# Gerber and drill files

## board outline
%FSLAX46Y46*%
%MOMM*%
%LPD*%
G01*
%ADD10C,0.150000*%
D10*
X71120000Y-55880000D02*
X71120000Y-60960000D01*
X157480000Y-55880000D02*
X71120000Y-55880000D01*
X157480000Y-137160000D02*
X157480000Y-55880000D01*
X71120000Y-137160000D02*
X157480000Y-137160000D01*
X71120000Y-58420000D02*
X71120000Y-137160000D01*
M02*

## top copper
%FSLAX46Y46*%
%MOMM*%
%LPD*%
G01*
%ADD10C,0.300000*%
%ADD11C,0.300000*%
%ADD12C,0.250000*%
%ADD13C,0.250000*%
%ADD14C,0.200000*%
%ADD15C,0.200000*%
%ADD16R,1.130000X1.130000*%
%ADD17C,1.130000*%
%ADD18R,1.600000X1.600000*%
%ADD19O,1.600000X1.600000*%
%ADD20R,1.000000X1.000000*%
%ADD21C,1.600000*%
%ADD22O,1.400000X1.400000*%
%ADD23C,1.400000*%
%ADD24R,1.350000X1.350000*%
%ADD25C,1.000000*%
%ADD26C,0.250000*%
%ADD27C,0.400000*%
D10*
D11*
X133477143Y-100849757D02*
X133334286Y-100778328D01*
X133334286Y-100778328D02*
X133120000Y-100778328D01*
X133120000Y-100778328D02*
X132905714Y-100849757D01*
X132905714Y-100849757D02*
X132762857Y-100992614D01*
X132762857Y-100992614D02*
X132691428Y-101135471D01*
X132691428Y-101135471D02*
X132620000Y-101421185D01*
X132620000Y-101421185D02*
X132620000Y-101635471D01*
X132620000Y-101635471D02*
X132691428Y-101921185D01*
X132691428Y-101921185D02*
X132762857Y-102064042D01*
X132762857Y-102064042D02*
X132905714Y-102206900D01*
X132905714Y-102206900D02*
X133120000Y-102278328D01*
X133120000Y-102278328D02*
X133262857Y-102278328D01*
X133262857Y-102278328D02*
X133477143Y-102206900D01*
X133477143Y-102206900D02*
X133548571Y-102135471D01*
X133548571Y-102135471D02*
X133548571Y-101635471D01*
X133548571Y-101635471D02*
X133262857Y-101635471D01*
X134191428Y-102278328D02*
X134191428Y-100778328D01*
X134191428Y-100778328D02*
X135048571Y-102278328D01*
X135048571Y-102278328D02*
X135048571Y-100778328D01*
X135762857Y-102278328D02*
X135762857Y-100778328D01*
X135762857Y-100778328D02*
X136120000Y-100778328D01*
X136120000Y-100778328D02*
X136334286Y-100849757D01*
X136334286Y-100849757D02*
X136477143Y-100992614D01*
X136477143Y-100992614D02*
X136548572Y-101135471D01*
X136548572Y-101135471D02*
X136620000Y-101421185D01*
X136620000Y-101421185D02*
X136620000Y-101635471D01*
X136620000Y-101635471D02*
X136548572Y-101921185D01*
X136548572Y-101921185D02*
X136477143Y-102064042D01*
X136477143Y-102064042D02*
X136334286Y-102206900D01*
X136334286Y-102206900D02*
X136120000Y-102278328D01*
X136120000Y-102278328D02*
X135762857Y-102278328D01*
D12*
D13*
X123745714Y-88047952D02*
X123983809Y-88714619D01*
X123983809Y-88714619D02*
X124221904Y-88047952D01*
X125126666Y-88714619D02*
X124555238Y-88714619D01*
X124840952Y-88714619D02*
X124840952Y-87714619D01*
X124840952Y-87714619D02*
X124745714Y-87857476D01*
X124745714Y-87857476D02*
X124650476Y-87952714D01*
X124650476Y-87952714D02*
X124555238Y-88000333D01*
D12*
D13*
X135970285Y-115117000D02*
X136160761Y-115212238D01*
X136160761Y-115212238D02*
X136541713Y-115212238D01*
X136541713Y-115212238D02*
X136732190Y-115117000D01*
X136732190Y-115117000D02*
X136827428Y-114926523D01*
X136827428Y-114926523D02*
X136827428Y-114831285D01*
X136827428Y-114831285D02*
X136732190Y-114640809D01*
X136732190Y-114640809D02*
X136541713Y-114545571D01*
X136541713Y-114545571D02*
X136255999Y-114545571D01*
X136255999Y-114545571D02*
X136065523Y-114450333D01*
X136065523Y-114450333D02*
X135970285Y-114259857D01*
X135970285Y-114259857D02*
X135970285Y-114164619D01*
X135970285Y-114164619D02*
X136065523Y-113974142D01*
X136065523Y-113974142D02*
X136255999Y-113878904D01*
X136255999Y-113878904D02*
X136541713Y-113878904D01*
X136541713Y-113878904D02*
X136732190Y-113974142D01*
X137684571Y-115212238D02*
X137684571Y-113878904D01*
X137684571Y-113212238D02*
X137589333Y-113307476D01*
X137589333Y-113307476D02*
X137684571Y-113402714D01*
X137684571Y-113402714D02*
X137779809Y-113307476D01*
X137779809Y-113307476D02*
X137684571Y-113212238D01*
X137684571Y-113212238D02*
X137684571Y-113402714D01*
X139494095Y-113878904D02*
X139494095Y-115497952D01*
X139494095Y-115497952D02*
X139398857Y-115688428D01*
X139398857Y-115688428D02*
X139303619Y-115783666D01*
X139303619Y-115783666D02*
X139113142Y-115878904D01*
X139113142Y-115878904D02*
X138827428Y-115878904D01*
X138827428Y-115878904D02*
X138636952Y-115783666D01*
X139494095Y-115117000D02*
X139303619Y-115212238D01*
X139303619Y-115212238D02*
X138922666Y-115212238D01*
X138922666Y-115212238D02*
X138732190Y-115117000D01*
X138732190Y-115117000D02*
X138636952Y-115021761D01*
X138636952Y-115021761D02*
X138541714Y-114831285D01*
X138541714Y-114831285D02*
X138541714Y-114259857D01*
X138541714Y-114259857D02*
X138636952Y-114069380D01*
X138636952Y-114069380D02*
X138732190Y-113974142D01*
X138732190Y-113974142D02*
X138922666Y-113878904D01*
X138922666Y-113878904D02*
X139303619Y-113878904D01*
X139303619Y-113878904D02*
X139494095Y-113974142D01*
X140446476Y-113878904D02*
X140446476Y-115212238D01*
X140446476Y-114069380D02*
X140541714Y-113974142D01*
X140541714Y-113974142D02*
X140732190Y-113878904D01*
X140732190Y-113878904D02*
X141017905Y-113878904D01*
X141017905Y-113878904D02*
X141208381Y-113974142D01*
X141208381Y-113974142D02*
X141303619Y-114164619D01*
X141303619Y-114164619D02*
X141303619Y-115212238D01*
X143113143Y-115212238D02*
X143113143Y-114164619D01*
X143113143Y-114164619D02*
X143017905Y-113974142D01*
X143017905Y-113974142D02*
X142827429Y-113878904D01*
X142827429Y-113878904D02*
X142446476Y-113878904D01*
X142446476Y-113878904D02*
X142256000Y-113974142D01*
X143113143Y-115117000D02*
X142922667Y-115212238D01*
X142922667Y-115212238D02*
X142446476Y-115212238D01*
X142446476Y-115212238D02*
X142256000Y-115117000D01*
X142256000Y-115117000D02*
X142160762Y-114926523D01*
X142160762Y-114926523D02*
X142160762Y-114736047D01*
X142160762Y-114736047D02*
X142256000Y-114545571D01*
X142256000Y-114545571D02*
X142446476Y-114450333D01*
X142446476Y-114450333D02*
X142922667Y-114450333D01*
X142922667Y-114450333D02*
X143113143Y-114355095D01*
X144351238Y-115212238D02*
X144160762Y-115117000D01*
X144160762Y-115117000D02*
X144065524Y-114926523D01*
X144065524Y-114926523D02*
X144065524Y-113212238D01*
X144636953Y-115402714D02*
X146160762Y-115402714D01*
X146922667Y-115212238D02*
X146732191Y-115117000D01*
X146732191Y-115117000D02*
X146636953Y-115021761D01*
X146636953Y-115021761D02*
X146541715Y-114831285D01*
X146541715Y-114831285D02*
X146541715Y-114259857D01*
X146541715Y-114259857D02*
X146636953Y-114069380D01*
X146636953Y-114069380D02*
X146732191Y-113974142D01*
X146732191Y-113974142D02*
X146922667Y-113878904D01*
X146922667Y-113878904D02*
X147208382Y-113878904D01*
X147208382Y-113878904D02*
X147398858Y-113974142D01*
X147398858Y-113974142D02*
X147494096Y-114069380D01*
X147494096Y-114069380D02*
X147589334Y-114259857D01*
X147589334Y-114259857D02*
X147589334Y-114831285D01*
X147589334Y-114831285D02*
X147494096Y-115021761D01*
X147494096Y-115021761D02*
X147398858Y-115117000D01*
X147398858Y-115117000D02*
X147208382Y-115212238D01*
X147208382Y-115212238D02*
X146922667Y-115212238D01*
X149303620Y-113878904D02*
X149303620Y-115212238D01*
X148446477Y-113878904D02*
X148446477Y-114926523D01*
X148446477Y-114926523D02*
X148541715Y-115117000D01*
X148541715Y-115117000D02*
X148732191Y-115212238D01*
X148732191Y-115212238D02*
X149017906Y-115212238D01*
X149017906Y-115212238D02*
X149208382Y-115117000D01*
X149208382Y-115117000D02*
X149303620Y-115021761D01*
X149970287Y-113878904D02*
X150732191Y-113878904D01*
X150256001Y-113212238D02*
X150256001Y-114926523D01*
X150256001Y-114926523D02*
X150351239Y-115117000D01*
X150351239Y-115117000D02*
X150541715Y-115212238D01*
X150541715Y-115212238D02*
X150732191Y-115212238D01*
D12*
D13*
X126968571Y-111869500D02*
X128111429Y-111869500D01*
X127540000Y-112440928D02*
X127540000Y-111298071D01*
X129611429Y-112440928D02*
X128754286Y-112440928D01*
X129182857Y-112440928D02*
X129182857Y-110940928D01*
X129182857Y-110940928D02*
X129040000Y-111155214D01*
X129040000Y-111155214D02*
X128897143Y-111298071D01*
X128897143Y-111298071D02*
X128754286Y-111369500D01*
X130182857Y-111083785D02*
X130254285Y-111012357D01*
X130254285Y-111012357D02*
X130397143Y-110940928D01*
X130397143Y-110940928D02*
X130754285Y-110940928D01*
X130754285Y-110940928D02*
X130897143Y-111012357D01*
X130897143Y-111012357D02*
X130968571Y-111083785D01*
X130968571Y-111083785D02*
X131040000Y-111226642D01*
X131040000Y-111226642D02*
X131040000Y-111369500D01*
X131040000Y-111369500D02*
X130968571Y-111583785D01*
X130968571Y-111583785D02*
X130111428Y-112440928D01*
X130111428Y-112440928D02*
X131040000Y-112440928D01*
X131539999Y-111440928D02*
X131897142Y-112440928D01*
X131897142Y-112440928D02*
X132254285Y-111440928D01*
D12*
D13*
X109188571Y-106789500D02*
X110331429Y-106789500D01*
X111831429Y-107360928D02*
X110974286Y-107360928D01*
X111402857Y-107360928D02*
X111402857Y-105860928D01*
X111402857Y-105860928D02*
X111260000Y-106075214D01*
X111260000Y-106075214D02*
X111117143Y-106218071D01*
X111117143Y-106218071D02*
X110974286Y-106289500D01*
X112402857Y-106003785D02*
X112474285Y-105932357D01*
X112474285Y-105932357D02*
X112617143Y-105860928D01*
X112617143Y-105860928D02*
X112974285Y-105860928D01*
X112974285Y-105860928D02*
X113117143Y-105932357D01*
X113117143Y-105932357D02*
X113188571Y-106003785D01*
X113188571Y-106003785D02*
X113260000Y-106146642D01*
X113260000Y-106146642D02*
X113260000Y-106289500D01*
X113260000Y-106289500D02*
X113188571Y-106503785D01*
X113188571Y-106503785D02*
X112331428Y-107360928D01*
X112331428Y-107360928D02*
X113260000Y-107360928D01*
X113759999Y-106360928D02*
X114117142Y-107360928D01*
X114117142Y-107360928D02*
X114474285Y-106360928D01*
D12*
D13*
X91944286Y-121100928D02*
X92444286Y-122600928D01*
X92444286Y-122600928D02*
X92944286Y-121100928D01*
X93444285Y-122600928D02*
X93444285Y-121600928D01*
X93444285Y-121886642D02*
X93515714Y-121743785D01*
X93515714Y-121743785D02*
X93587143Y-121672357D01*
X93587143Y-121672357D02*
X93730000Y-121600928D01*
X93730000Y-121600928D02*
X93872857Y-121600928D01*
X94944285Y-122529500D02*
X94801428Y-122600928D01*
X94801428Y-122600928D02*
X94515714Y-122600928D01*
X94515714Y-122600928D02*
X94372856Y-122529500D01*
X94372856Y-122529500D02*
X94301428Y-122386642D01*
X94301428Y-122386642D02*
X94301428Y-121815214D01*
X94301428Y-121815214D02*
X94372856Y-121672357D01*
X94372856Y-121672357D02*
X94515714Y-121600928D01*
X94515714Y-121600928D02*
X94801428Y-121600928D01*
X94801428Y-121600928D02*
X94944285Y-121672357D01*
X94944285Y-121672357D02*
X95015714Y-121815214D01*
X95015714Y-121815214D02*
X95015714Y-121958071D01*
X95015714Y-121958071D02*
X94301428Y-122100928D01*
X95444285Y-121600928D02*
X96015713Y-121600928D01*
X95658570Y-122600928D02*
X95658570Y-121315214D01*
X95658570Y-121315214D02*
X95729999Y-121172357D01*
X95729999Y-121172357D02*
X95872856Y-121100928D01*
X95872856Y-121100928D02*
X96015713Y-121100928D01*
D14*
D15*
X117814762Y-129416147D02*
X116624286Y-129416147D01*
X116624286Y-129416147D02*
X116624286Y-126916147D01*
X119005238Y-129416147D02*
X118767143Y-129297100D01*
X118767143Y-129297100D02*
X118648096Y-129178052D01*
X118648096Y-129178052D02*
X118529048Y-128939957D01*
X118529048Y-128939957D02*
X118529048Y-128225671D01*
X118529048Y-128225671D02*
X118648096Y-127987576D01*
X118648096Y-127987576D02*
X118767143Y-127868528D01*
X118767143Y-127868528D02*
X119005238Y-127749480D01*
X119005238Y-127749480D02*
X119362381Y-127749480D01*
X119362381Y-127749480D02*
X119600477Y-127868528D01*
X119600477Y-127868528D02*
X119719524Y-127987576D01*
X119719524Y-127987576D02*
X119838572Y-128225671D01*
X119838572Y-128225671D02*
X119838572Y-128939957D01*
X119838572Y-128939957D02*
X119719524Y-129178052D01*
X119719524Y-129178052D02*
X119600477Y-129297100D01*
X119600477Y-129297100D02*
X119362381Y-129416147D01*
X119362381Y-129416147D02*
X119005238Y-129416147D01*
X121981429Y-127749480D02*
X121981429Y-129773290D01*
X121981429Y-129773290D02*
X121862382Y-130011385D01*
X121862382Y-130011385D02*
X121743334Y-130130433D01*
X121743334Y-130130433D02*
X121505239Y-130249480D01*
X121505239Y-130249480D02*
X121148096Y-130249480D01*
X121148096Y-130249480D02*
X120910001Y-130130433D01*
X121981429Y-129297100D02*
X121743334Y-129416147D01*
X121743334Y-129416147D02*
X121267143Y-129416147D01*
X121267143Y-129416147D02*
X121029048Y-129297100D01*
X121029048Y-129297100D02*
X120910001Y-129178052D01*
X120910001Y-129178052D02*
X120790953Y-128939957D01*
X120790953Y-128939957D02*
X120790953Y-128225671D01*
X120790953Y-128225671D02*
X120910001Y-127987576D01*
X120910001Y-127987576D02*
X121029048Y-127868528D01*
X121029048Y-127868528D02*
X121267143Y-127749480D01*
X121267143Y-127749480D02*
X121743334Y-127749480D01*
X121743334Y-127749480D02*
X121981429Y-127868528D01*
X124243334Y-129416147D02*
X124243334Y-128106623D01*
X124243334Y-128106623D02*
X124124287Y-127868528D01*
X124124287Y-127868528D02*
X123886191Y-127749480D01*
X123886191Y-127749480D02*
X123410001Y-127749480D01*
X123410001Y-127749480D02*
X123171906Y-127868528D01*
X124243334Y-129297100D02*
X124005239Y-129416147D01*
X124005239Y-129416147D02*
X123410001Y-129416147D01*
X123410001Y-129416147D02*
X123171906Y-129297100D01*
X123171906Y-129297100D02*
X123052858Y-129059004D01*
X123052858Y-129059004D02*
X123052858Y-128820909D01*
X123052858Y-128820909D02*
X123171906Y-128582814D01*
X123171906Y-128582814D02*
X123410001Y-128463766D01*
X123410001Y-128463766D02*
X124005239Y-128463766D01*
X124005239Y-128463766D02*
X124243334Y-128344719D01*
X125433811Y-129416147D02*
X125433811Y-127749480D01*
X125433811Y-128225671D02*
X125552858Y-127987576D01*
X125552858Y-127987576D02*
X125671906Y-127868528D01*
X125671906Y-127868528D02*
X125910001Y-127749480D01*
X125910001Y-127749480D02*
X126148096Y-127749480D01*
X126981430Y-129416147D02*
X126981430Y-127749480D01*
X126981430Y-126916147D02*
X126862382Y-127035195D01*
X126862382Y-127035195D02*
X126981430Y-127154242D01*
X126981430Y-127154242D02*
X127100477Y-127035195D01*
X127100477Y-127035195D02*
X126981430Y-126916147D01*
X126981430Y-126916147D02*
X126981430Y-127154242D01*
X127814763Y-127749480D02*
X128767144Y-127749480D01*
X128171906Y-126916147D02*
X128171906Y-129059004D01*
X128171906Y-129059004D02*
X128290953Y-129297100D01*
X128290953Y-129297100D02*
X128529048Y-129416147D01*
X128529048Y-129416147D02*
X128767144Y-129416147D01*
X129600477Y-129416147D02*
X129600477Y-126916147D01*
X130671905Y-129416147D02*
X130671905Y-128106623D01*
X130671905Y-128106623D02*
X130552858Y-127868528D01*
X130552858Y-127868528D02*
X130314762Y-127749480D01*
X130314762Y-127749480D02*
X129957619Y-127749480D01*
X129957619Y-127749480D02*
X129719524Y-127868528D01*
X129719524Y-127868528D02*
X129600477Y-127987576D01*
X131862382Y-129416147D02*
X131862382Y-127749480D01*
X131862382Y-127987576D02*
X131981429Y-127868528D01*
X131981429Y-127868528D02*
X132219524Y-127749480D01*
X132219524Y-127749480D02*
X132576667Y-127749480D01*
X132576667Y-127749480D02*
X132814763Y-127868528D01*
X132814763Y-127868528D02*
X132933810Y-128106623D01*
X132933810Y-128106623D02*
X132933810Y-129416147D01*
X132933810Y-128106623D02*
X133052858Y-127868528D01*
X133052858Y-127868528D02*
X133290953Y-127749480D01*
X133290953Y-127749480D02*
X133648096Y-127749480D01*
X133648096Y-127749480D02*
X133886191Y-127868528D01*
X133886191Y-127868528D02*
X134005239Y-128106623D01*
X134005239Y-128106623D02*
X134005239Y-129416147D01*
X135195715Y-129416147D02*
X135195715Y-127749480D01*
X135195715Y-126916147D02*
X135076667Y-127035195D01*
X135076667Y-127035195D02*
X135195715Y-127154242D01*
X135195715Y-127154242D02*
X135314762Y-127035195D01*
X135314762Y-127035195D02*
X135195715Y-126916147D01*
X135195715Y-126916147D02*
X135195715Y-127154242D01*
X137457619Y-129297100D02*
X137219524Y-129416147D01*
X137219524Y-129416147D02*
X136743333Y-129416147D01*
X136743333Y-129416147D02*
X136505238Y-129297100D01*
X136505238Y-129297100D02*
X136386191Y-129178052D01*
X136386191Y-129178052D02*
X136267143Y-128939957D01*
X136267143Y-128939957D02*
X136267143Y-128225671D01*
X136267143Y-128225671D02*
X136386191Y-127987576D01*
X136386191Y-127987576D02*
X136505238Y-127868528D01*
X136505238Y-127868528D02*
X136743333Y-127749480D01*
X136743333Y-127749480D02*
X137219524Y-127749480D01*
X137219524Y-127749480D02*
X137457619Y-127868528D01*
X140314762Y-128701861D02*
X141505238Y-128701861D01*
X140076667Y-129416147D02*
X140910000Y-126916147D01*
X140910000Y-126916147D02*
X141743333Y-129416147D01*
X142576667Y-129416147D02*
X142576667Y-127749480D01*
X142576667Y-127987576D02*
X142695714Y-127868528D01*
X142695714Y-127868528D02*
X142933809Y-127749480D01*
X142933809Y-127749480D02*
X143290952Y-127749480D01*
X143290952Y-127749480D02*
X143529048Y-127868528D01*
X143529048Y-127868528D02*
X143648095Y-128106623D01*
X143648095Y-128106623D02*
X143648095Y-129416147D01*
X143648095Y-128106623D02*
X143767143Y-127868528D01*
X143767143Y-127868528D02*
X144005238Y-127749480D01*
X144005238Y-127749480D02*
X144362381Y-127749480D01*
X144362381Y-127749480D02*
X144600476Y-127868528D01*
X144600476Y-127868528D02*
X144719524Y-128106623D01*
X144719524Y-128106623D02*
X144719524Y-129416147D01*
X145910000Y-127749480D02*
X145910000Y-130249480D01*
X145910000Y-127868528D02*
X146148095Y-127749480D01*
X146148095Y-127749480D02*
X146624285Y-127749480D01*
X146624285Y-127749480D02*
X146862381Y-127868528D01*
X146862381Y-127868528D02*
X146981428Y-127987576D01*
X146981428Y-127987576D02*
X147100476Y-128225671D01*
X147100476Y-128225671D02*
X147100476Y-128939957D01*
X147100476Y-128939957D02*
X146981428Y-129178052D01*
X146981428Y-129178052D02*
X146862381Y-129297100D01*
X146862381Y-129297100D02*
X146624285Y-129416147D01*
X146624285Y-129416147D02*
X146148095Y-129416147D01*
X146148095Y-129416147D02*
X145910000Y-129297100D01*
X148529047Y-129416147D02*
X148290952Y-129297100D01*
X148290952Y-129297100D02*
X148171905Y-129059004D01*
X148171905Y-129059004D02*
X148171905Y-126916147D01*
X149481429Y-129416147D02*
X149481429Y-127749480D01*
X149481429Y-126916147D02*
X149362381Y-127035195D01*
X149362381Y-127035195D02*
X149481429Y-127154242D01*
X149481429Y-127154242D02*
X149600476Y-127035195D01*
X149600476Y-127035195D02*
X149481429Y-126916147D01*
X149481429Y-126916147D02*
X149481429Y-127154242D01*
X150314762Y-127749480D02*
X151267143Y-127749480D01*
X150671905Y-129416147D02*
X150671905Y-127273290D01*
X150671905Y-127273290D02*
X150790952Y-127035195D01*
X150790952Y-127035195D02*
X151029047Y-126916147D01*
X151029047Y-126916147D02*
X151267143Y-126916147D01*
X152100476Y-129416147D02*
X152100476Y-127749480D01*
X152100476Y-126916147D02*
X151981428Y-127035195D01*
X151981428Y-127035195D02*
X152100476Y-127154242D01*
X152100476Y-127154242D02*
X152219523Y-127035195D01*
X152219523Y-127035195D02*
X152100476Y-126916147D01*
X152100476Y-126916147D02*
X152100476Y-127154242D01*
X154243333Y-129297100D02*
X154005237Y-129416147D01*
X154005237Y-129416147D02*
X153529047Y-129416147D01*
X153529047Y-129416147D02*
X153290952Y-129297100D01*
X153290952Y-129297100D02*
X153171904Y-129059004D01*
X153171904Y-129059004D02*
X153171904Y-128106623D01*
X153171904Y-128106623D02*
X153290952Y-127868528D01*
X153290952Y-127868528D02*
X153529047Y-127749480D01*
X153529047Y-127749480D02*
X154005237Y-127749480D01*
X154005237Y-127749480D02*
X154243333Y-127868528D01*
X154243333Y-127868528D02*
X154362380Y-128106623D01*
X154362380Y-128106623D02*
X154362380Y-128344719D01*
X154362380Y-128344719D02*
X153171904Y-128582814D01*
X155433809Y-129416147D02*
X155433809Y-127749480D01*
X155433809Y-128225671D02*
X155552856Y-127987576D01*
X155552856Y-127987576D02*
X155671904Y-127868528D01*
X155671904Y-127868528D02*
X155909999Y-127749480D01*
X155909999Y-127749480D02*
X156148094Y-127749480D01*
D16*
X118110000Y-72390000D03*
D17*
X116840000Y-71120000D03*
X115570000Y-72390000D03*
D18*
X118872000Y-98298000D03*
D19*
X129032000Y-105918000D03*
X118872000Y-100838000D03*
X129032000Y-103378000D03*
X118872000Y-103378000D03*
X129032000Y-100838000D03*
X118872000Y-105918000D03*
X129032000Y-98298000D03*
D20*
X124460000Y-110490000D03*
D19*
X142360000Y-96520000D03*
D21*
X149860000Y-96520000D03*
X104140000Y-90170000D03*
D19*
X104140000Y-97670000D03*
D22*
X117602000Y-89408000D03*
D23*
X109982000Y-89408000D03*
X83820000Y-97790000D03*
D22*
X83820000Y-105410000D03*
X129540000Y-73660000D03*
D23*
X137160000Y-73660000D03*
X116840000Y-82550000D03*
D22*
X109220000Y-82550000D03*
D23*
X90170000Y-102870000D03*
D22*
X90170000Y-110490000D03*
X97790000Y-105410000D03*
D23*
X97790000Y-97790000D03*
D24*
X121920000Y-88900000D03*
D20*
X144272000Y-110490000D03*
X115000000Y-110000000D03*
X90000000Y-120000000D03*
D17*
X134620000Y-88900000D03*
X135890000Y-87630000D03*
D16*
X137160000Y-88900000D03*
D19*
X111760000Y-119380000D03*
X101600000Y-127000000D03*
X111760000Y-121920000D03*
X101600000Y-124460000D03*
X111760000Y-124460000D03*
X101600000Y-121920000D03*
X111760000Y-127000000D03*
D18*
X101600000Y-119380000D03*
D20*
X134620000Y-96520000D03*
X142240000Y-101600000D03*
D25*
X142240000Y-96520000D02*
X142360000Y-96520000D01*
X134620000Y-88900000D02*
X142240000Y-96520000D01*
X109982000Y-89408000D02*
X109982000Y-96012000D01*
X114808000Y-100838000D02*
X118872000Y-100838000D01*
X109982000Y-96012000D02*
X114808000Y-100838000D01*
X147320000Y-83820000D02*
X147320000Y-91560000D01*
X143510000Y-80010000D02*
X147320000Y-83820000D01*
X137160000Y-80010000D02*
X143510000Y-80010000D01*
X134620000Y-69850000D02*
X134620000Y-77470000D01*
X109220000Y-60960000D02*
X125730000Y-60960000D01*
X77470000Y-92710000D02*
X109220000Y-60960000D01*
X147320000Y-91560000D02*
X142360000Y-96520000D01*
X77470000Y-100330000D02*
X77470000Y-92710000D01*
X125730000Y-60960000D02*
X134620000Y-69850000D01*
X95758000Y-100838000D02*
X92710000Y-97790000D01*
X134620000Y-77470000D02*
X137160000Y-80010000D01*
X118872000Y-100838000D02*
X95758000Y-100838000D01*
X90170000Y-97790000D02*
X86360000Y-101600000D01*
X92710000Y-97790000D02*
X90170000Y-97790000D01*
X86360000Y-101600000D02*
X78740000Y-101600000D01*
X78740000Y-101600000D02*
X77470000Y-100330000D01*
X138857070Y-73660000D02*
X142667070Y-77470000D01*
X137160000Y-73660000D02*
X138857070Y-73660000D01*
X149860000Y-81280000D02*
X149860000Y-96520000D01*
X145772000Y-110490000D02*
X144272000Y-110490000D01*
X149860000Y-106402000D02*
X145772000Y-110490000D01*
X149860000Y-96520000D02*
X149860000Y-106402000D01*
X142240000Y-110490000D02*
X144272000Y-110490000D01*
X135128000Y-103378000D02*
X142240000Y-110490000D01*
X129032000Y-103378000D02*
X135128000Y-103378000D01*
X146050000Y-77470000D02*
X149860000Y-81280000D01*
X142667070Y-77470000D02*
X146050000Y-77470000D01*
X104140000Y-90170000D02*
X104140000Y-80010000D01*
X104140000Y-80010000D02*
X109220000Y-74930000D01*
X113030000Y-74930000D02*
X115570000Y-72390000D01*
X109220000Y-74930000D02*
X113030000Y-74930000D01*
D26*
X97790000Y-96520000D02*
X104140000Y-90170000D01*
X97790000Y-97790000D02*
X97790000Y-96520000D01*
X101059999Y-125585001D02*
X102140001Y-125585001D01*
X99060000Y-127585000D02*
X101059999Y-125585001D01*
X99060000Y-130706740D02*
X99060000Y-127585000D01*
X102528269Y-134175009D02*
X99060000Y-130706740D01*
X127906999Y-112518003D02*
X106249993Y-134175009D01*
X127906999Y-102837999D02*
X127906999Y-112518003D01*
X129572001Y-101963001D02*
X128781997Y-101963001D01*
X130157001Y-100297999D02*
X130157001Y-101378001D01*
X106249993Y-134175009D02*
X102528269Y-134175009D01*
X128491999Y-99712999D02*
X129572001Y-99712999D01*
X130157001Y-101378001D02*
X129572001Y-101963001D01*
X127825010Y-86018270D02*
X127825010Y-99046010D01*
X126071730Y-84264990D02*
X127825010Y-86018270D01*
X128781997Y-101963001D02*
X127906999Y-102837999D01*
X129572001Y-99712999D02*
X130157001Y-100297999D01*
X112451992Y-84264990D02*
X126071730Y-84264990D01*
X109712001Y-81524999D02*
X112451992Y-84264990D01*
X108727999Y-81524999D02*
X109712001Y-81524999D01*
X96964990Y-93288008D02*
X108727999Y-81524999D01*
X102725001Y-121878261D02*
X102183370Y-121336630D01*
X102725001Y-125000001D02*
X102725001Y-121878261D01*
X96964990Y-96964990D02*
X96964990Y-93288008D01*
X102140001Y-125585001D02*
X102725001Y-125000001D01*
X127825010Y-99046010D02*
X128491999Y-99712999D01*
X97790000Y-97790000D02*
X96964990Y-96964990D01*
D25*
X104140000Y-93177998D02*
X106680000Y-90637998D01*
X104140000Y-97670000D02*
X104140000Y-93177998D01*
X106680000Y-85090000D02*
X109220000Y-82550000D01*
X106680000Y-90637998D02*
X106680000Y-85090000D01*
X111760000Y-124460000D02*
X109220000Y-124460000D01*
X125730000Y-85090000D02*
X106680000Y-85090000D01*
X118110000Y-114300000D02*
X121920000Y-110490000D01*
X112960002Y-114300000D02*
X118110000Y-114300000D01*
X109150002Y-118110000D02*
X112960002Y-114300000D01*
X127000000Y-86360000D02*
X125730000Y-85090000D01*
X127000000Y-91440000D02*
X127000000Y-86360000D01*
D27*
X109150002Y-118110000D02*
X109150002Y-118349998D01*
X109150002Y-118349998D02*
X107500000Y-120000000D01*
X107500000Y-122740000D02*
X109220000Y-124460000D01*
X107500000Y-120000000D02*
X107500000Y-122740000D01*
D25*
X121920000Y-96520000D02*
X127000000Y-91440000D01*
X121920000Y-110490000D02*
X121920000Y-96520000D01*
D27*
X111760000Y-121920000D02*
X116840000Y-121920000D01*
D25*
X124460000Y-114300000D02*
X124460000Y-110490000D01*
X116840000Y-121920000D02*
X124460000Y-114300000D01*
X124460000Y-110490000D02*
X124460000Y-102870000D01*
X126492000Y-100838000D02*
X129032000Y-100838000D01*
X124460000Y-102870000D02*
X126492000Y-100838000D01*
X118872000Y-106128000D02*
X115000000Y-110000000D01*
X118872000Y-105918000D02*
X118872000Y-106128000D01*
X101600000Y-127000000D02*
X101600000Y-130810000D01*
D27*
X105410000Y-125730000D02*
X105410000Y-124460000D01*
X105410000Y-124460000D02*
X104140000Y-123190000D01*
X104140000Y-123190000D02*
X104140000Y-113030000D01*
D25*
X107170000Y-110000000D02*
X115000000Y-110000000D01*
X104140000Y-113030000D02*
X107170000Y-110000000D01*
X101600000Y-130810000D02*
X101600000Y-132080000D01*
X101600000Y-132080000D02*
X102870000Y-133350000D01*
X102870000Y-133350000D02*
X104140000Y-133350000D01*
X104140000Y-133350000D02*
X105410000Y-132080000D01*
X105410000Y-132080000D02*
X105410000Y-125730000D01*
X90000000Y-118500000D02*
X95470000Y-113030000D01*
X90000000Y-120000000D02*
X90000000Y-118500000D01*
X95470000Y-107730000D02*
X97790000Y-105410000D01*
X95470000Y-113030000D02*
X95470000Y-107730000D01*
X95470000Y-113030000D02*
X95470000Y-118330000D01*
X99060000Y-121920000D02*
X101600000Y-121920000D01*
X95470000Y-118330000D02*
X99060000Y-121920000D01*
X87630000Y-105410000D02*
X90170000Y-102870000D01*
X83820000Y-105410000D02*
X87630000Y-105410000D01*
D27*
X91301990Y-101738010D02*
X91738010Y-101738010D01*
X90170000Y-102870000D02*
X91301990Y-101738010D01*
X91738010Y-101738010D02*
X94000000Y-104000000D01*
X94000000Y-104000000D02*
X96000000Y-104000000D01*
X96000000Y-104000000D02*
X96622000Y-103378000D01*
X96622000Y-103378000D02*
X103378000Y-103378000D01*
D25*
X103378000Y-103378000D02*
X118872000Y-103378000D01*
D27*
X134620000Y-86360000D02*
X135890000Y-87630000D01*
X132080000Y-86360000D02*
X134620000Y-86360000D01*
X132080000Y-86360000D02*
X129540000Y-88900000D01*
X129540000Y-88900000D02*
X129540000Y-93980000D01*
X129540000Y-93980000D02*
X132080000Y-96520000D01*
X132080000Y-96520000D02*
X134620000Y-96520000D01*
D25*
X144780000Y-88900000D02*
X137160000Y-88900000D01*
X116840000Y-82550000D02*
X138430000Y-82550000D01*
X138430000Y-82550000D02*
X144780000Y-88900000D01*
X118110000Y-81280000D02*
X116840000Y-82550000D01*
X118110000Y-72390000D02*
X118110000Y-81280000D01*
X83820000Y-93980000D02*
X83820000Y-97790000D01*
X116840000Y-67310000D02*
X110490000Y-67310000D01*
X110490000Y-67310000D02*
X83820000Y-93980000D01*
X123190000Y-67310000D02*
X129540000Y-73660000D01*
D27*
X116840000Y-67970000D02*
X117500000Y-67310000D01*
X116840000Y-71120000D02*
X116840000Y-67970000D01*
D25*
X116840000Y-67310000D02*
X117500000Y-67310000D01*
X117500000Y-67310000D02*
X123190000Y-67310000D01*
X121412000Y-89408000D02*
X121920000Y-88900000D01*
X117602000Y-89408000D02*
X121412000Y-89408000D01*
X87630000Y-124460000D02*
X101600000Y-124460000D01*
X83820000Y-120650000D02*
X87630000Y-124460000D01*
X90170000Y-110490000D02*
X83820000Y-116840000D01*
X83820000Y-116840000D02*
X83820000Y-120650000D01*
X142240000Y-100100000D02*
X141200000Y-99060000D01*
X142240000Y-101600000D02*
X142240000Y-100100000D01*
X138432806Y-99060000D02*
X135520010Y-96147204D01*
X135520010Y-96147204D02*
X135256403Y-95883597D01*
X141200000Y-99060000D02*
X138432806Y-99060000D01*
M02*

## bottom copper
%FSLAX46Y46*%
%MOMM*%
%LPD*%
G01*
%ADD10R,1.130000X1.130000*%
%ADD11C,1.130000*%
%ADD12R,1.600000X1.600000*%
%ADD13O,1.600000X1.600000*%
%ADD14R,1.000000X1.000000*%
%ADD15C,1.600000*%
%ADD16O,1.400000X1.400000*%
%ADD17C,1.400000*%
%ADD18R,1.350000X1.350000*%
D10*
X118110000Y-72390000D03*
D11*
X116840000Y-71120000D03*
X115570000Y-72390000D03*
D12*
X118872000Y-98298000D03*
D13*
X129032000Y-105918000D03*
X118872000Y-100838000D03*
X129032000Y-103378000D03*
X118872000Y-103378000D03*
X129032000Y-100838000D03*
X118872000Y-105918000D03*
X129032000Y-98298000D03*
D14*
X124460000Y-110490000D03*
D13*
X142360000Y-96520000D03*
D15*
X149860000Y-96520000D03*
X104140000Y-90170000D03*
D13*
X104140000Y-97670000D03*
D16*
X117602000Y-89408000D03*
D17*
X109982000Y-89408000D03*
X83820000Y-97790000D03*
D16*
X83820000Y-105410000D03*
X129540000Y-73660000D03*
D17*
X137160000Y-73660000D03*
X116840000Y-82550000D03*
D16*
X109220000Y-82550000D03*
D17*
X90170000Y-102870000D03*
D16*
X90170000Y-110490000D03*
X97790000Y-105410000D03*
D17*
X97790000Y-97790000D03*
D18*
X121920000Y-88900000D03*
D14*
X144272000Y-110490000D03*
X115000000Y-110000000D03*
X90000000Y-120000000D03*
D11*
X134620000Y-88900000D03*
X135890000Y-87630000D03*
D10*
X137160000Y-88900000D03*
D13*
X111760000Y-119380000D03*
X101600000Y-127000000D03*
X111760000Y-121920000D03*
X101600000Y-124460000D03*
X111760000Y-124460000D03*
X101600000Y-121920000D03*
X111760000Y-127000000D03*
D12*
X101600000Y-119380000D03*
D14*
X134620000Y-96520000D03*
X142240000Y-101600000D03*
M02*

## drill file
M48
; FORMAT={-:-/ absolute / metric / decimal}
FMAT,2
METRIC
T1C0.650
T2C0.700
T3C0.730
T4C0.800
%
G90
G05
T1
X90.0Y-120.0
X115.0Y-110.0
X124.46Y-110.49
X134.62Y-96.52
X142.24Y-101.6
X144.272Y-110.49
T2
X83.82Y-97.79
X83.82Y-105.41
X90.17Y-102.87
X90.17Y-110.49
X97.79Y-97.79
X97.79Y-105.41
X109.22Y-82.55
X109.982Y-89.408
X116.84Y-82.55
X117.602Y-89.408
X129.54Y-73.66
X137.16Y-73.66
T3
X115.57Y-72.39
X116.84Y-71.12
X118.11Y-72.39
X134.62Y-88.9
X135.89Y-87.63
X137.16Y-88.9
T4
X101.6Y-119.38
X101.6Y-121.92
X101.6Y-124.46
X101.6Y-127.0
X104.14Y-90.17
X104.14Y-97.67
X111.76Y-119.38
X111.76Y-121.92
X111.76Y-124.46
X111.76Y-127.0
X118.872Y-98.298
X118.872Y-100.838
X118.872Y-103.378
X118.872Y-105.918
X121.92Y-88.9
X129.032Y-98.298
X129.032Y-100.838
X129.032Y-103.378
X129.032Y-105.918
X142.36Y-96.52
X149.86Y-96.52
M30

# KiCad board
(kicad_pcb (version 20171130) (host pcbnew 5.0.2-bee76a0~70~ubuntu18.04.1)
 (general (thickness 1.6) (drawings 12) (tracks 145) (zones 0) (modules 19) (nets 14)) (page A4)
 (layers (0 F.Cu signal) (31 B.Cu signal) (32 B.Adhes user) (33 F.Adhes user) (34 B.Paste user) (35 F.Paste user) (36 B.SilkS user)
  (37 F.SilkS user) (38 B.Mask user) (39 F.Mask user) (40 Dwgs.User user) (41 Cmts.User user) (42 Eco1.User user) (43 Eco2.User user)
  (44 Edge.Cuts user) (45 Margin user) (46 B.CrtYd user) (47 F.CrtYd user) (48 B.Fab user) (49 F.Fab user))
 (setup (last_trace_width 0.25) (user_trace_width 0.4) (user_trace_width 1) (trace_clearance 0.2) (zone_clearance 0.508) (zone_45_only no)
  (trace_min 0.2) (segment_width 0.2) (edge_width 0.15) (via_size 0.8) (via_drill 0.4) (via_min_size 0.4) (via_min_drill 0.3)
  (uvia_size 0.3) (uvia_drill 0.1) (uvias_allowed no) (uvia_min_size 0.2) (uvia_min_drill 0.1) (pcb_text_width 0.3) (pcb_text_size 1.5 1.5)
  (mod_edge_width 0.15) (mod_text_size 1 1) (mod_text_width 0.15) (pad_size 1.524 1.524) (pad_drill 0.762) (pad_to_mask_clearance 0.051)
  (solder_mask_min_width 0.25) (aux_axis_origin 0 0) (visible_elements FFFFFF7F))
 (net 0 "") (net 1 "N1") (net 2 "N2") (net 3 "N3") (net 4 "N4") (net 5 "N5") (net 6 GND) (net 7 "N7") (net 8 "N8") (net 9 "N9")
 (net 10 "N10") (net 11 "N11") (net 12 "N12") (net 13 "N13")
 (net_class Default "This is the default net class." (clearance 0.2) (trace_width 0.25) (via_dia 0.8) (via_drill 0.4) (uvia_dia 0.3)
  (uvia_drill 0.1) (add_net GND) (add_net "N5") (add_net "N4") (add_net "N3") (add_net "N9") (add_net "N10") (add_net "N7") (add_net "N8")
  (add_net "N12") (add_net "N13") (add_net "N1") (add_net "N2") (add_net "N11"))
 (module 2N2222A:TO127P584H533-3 (layer F.Cu) (at 116.84 72.39 180)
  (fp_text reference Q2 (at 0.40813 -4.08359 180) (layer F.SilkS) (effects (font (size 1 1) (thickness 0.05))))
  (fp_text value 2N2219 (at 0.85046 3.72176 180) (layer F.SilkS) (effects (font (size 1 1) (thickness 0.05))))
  (pad 1 thru_hole rect (at -1.27 0 180) (size 1.13 1.13) (drill 0.73) (layers *.Cu *.Mask) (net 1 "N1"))
  (pad 2 thru_hole circle (at 0 1.27 180) (size 1.13 1.13) (drill 0.73) (layers *.Cu *.Mask) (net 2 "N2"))
  (pad 3 thru_hole circle (at 1.27 0 180) (size 1.13 1.13) (drill 0.73) (layers *.Cu *.Mask) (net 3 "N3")))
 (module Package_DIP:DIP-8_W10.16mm (layer F.Cu) (at 118.872 98.298)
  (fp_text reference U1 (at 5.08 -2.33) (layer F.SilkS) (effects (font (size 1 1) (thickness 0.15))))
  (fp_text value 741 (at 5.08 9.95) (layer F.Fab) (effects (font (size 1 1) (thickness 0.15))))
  (pad 1 thru_hole rect (at 0 0) (size 1.6 1.6) (drill 0.8) (layers *.Cu *.Mask))
  (pad 5 thru_hole oval (at 10.16 7.62) (size 1.6 1.6) (drill 0.8) (layers *.Cu *.Mask))
  (pad 2 thru_hole oval (at 0 2.54) (size 1.6 1.6) (drill 0.8) (layers *.Cu *.Mask) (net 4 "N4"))
  (pad 6 thru_hole oval (at 10.16 5.08) (size 1.6 1.6) (drill 0.8) (layers *.Cu *.Mask) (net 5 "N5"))
  (pad 3 thru_hole oval (at 0 5.08) (size 1.6 1.6) (drill 0.8) (layers *.Cu *.Mask) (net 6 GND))
  (pad 7 thru_hole oval (at 10.16 2.54) (size 1.6 1.6) (drill 0.8) (layers *.Cu *.Mask) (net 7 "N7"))
  (pad 4 thru_hole oval (at 0 7.62) (size 1.6 1.6) (drill 0.8) (layers *.Cu *.Mask) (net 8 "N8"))
  (pad 8 thru_hole oval (at 10.16 0) (size 1.6 1.6) (drill 0.8) (layers *.Cu *.Mask)))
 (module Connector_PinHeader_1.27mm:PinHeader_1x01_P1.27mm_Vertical (layer F.Cu) (at 124.46 110.49)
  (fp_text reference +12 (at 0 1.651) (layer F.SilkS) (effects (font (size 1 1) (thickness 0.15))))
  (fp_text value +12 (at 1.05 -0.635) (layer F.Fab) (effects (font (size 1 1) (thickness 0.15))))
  (pad 1 thru_hole rect (at 0 0) (size 1 1) (drill 0.65) (layers *.Cu *.Mask) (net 7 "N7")))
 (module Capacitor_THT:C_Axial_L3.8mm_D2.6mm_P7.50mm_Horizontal (layer F.Cu) (at 149.86 96.52 180)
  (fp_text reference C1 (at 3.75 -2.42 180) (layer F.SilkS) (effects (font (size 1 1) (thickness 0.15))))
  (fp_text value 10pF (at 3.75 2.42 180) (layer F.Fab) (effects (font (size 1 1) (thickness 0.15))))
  (pad 2 thru_hole oval (at 7.5 0 180) (size 1.6 1.6) (drill 0.8) (layers *.Cu *.Mask) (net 4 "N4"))
  (pad 1 thru_hole circle (at 0 0 180) (size 1.6 1.6) (drill 0.8) (layers *.Cu *.Mask) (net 5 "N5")))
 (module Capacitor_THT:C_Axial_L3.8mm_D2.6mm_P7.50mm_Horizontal (layer F.Cu) (at 104.14 90.17 270)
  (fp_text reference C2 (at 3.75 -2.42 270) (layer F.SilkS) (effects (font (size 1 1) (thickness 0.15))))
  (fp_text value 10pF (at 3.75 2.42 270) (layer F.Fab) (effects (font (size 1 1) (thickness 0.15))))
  (pad 1 thru_hole circle (at 0 0 270) (size 1.6 1.6) (drill 0.8) (layers *.Cu *.Mask) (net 3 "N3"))
  (pad 2 thru_hole oval (at 7.5 0 270) (size 1.6 1.6) (drill 0.8) (layers *.Cu *.Mask) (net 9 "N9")))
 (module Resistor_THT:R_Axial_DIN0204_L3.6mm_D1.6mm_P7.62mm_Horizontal (layer F.Cu) (at 109.982 89.408)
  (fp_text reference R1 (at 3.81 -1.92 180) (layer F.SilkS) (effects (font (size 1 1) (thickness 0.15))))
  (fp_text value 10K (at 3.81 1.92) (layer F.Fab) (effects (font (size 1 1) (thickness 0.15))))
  (pad 2 thru_hole oval (at 7.62 0) (size 1.4 1.4) (drill 0.7) (layers *.Cu *.Mask) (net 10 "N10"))
  (pad 1 thru_hole circle (at 0 0) (size 1.4 1.4) (drill 0.7) (layers *.Cu *.Mask) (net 4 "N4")))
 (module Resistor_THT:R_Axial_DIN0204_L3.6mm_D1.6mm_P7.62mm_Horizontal (layer F.Cu) (at 83.82 97.79 270)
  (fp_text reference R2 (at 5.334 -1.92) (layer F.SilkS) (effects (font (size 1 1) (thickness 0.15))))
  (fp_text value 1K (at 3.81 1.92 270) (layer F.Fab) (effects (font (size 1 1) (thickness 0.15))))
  (pad 1 thru_hole circle (at 0 0 270) (size 1.4 1.4) (drill 0.7) (layers *.Cu *.Mask) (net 2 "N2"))
  (pad 2 thru_hole oval (at 7.62 0 270) (size 1.4 1.4) (drill 0.7) (layers *.Cu *.Mask) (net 6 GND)))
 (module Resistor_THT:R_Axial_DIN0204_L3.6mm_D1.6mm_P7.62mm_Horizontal (layer F.Cu) (at 137.16 73.66 180)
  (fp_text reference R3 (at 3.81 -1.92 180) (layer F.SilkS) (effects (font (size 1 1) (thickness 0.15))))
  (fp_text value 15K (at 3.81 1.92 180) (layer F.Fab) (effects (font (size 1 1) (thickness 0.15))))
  (pad 2 thru_hole oval (at 7.62 0 180) (size 1.4 1.4) (drill 0.7) (layers *.Cu *.Mask) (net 2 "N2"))
  (pad 1 thru_hole circle (at 0 0 180) (size 1.4 1.4) (drill 0.7) (layers *.Cu *.Mask) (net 5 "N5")))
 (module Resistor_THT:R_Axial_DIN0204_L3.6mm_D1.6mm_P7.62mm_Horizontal (layer F.Cu) (at 116.84 82.55 180)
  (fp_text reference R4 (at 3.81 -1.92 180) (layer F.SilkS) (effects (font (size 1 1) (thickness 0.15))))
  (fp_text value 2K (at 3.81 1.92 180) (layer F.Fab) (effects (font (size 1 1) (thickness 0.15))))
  (pad 1 thru_hole circle (at 0 0 180) (size 1.4 1.4) (drill 0.7) (layers *.Cu *.Mask) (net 1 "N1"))
  (pad 2 thru_hole oval (at 7.62 0 180) (size 1.4 1.4) (drill 0.7) (layers *.Cu *.Mask) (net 9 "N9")))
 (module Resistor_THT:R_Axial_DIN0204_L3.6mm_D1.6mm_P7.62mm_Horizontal (layer F.Cu) (at 90.17 102.87 270)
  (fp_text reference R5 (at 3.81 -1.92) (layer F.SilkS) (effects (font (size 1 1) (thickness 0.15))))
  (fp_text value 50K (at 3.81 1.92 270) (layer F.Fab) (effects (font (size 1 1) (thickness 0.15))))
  (pad 1 thru_hole circle (at 0 0 270) (size 1.4 1.4) (drill 0.7) (layers *.Cu *.Mask) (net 6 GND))
  (pad 2 thru_hole oval (at 7.62 0 270) (size 1.4 1.4) (drill 0.7) (layers *.Cu *.Mask) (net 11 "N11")))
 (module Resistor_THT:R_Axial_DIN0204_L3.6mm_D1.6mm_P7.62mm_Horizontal (layer F.Cu) (at 97.79 97.79 270)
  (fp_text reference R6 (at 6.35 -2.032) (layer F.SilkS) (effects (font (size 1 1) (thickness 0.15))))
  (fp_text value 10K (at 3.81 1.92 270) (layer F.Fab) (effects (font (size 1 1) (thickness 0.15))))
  (pad 2 thru_hole oval (at 7.62 0 270) (size 1.4 1.4) (drill 0.7) (layers *.Cu *.Mask) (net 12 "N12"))
  (pad 1 thru_hole circle (at 0 0 270) (size 1.4 1.4) (drill 0.7) (layers *.Cu *.Mask) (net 3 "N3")))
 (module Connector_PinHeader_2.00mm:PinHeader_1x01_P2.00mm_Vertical (layer F.Cu) (at 121.92 88.9)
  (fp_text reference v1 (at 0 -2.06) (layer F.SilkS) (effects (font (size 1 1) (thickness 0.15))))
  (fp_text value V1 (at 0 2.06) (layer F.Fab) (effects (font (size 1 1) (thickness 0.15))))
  (pad 1 thru_hole rect (at 0 0) (size 1.35 1.35) (drill 0.8) (layers *.Cu *.Mask) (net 10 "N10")))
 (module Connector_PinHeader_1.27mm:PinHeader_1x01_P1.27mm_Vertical (layer F.Cu) (at 144.272 110.49)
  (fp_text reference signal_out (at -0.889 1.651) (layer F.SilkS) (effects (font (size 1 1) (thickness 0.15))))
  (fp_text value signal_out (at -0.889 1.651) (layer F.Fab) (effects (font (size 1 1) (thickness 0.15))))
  (pad 1 thru_hole rect (at 0 0) (size 1 1) (drill 0.65) (layers *.Cu *.Mask) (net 5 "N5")))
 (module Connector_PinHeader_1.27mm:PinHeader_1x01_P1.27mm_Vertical (layer F.Cu) (at 115 110)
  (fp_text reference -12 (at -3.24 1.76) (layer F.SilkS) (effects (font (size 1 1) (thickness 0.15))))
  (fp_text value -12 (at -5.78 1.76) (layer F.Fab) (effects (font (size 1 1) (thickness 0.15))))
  (pad 1 thru_hole rect (at 0 0) (size 1 1) (drill 0.65) (layers *.Cu *.Mask) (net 8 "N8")))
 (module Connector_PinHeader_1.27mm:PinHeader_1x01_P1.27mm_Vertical (layer F.Cu) (at 90 120)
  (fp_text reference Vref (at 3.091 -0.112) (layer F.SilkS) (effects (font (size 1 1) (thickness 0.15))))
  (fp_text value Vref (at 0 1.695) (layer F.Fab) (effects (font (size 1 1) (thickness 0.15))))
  (pad 1 thru_hole rect (at 0 0) (size 1 1) (drill 0.65) (layers *.Cu *.Mask) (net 12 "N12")))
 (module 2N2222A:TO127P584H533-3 (layer F.Cu) (at 135.89 88.9 180)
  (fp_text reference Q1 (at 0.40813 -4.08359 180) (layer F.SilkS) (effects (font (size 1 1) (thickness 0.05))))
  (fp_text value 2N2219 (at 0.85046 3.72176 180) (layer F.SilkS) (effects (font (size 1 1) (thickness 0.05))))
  (pad 3 thru_hole circle (at 1.27 0 180) (size 1.13 1.13) (drill 0.73) (layers *.Cu *.Mask) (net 4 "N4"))
  (pad 2 thru_hole circle (at 0 1.27 180) (size 1.13 1.13) (drill 0.73) (layers *.Cu *.Mask) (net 6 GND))
  (pad 1 thru_hole rect (at -1.27 0 180) (size 1.13 1.13) (drill 0.73) (layers *.Cu *.Mask) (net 1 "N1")))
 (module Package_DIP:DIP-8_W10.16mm (layer F.Cu) (at 101.6 119.38)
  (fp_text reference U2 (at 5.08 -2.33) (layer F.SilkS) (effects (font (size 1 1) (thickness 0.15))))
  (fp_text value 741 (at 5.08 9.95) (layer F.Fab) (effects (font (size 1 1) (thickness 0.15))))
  (pad 8 thru_hole oval (at 10.16 0) (size 1.6 1.6) (drill 0.8) (layers *.Cu *.Mask))
  (pad 4 thru_hole oval (at 0 7.62) (size 1.6 1.6) (drill 0.8) (layers *.Cu *.Mask) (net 8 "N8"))
  (pad 7 thru_hole oval (at 10.16 2.54) (size 1.6 1.6) (drill 0.8) (layers *.Cu *.Mask) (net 7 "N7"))
  (pad 3 thru_hole oval (at 0 5.08) (size 1.6 1.6) (drill 0.8) (layers *.Cu *.Mask) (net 11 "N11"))
  (pad 6 thru_hole oval (at 10.16 5.08) (size 1.6 1.6) (drill 0.8) (layers *.Cu *.Mask) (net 9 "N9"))
  (pad 2 thru_hole oval (at 0 2.54) (size 1.6 1.6) (drill 0.8) (layers *.Cu *.Mask) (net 3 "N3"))
  (pad 5 thru_hole oval (at 10.16 7.62) (size 1.6 1.6) (drill 0.8) (layers *.Cu *.Mask))
  (pad 1 thru_hole rect (at 0 0) (size 1.6 1.6) (drill 0.8) (layers *.Cu *.Mask)))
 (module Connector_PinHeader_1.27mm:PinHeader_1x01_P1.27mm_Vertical (layer F.Cu) (at 134.62 96.52)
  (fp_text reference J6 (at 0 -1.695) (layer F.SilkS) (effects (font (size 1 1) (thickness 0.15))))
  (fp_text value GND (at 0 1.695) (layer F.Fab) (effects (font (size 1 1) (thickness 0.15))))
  (pad 1 thru_hole rect (at 0 0) (size 1 1) (drill 0.65) (layers *.Cu *.Mask) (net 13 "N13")))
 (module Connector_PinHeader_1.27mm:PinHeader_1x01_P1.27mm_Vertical (layer F.Cu) (at 142.24 101.6)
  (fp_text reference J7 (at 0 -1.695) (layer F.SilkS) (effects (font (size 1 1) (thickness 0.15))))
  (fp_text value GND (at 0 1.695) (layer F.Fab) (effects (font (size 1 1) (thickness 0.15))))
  (pad 1 thru_hole rect (at 0 0) (size 1 1) (drill 0.65) (layers *.Cu *.Mask) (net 13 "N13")))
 (gr_line (start 71.12 55.88) (end 71.12 60.96) (layer Edge.Cuts) (width 0.15))
 (gr_line (start 157.48 55.88) (end 71.12 55.88) (layer Edge.Cuts) (width 0.15))
 (gr_line (start 157.48 137.16) (end 157.48 55.88) (layer Edge.Cuts) (width 0.15))
 (gr_line (start 71.12 137.16) (end 157.48 137.16) (layer Edge.Cuts) (width 0.15))
 (gr_line (start 71.12 58.42) (end 71.12 137.16) (layer Edge.Cuts) (width 0.15))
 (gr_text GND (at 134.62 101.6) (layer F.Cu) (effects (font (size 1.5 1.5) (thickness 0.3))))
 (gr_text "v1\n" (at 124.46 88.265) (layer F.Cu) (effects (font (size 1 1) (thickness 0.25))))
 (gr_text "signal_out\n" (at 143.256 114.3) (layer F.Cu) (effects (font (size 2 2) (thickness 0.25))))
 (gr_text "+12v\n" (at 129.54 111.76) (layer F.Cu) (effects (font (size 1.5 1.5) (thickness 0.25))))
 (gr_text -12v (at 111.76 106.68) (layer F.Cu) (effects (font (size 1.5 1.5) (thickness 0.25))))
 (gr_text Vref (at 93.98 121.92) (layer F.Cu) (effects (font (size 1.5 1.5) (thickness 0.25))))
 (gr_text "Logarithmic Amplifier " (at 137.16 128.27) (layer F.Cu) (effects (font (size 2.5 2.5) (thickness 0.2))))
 (segment (start 142.24 96.52) (end 142.36 96.52) (width 1) (layer F.Cu) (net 4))
 (segment (start 134.62 88.9) (end 142.24 96.52) (width 1) (layer F.Cu) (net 4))
 (segment (start 109.982 89.408) (end 109.982 96.012) (width 1) (layer F.Cu) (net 4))
 (segment (start 114.808 100.838) (end 118.872 100.838) (width 1) (layer F.Cu) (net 4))
 (segment (start 109.982 96.012) (end 114.808 100.838) (width 1) (layer F.Cu) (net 4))
 (segment (start 147.32 83.82) (end 147.32 91.56) (width 1) (layer F.Cu) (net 4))
 (segment (start 143.51 80.01) (end 147.32 83.82) (width 1) (layer F.Cu) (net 4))
 (segment (start 137.16 80.01) (end 143.51 80.01) (width 1) (layer F.Cu) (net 4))
 (segment (start 134.62 69.85) (end 134.62 77.47) (width 1) (layer F.Cu) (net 4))
 (segment (start 109.22 60.96) (end 125.73 60.96) (width 1) (layer F.Cu) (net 4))
 (segment (start 77.47 92.71) (end 109.22 60.96) (width 1) (layer F.Cu) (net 4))
 (segment (start 147.32 91.56) (end 142.36 96.52) (width 1) (layer F.Cu) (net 4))
 (segment (start 77.47 100.33) (end 77.47 92.71) (width 1) (layer F.Cu) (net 4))
 (segment (start 125.73 60.96) (end 134.62 69.85) (width 1) (layer F.Cu) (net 4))
 (segment (start 95.758 100.838) (end 92.71 97.79) (width 1) (layer F.Cu) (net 4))
 (segment (start 134.62 77.47) (end 137.16 80.01) (width 1) (layer F.Cu) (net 4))
 (segment (start 118.872 100.838) (end 95.758 100.838) (width 1) (layer F.Cu) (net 4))
 (segment (start 90.17 97.79) (end 86.36 101.6) (width 1) (layer F.Cu) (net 4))
 (segment (start 92.71 97.79) (end 90.17 97.79) (width 1) (layer F.Cu) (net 4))
 (segment (start 86.36 101.6) (end 78.74 101.6) (width 1) (layer F.Cu) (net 4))
 (segment (start 78.74 101.6) (end 77.47 100.33) (width 1) (layer F.Cu) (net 4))
 (segment (start 138.85707 73.66) (end 142.66707 77.47) (width 1) (layer F.Cu) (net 5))
 (segment (start 137.16 73.66) (end 138.85707 73.66) (width 1) (layer F.Cu) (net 5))
 (segment (start 149.86 81.28) (end 149.86 96.52) (width 1) (layer F.Cu) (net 5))
 (segment (start 145.772 110.49) (end 144.272 110.49) (width 1) (layer F.Cu) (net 5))
 (segment (start 149.86 106.402) (end 145.772 110.49) (width 1) (layer F.Cu) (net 5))
 (segment (start 149.86 96.52) (end 149.86 106.402) (width 1) (layer F.Cu) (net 5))
 (segment (start 142.24 110.49) (end 144.272 110.49) (width 1) (layer F.Cu) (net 5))
 (segment (start 135.128 103.378) (end 142.24 110.49) (width 1) (layer F.Cu) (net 5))
 (segment (start 129.032 103.378) (end 135.128 103.378) (width 1) (layer F.Cu) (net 5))
 (segment (start 146.05 77.47) (end 149.86 81.28) (width 1) (layer F.Cu) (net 5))
 (segment (start 142.66707 77.47) (end 146.05 77.47) (width 1) (layer F.Cu) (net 5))
 (segment (start 104.14 90.17) (end 104.14 80.01) (width 1) (layer F.Cu) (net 3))
 (segment (start 104.14 80.01) (end 109.22 74.93) (width 1) (layer F.Cu) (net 3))
 (segment (start 113.03 74.93) (end 115.57 72.39) (width 1) (layer F.Cu) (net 3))
 (segment (start 109.22 74.93) (end 113.03 74.93) (width 1) (layer F.Cu) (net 3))
 (segment (start 97.79 96.52) (end 104.14 90.17) (width 0.25) (layer F.Cu) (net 3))
 (segment (start 97.79 97.79) (end 97.79 96.52) (width 0.25) (layer F.Cu) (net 3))
 (segment (start 101.059999 125.585001) (end 102.140001 125.585001) (width 0.25) (layer F.Cu) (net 3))
 (segment (start 99.06 127.585) (end 101.059999 125.585001) (width 0.25) (layer F.Cu) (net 3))
 (segment (start 99.06 130.70674) (end 99.06 127.585) (width 0.25) (layer F.Cu) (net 3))
 (segment (start 102.528269 134.175009) (end 99.06 130.70674) (width 0.25) (layer F.Cu) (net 3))
 (segment (start 127.906999 112.518003) (end 106.249993 134.175009) (width 0.25) (layer F.Cu) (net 3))
 (segment (start 127.906999 102.837999) (end 127.906999 112.518003) (width 0.25) (layer F.Cu) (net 3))
 (segment (start 129.572001 101.963001) (end 128.781997 101.963001) (width 0.25) (layer F.Cu) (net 3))
 (segment (start 130.157001 100.297999) (end 130.157001 101.378001) (width 0.25) (layer F.Cu) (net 3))
 (segment (start 106.249993 134.175009) (end 102.528269 134.175009) (width 0.25) (layer F.Cu) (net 3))
 (segment (start 128.491999 99.712999) (end 129.572001 99.712999) (width 0.25) (layer F.Cu) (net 3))
 (segment (start 130.157001 101.378001) (end 129.572001 101.963001) (width 0.25) (layer F.Cu) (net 3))
 (segment (start 127.82501 86.01827) (end 127.82501 99.04601) (width 0.25) (layer F.Cu) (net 3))
 (segment (start 126.07173 84.26499) (end 127.82501 86.01827) (width 0.25) (layer F.Cu) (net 3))
 (segment (start 128.781997 101.963001) (end 127.906999 102.837999) (width 0.25) (layer F.Cu) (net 3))
 (segment (start 129.572001 99.712999) (end 130.157001 100.297999) (width 0.25) (layer F.Cu) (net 3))
 (segment (start 112.451992 84.26499) (end 126.07173 84.26499) (width 0.25) (layer F.Cu) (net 3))
 (segment (start 109.712001 81.524999) (end 112.451992 84.26499) (width 0.25) (layer F.Cu) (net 3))
 (segment (start 108.727999 81.524999) (end 109.712001 81.524999) (width 0.25) (layer F.Cu) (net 3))
 (segment (start 96.96499 93.288008) (end 108.727999 81.524999) (width 0.25) (layer F.Cu) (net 3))
 (segment (start 102.725001 121.878261) (end 102.18337 121.33663) (width 0.25) (layer F.Cu) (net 3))
 (segment (start 102.725001 125.000001) (end 102.725001 121.878261) (width 0.25) (layer F.Cu) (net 3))
 (segment (start 96.96499 96.96499) (end 96.96499 93.288008) (width 0.25) (layer F.Cu) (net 3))
 (segment (start 102.140001 125.585001) (end 102.725001 125.000001) (width 0.25) (layer F.Cu) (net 3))
 (segment (start 127.82501 99.04601) (end 128.491999 99.712999) (width 0.25) (layer F.Cu) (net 3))
 (segment (start 97.79 97.79) (end 96.96499 96.96499) (width 0.25) (layer F.Cu) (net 3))
 (segment (start 104.14 93.177998) (end 106.68 90.637998) (width 1) (layer F.Cu) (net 9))
 (segment (start 104.14 97.67) (end 104.14 93.177998) (width 1) (layer F.Cu) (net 9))
 (segment (start 106.68 85.09) (end 109.22 82.55) (width 1) (layer F.Cu) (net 9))
 (segment (start 106.68 90.637998) (end 106.68 85.09) (width 1) (layer F.Cu) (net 9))
 (segment (start 111.76 124.46) (end 109.22 124.46) (width 1) (layer F.Cu) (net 9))
 (segment (start 125.73 85.09) (end 106.68 85.09) (width 1) (layer F.Cu) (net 9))
 (segment (start 118.11 114.3) (end 121.92 110.49) (width 1) (layer F.Cu) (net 9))
 (segment (start 112.960002 114.3) (end 118.11 114.3) (width 1) (layer F.Cu) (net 9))
 (segment (start 109.150002 118.11) (end 112.960002 114.3) (width 1) (layer F.Cu) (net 9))
 (segment (start 127 86.36) (end 125.73 85.09) (width 1) (layer F.Cu) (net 9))
 (segment (start 127 91.44) (end 127 86.36) (width 1) (layer F.Cu) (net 9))
 (segment (start 109.150002 118.11) (end 109.150002 118.349998) (width 0.4) (layer F.Cu) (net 9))
 (segment (start 109.150002 118.349998) (end 107.5 120) (width 0.4) (layer F.Cu) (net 9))
 (segment (start 107.5 122.74) (end 109.22 124.46) (width 0.4) (layer F.Cu) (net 9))
 (segment (start 107.5 120) (end 107.5 122.74) (width 0.4) (layer F.Cu) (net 9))
 (segment (start 121.92 96.52) (end 127 91.44) (width 1) (layer F.Cu) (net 9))
 (segment (start 121.92 110.49) (end 121.92 96.52) (width 1) (layer F.Cu) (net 9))
 (segment (start 111.76 121.92) (end 116.84 121.92) (width 0.4) (layer F.Cu) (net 7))
 (segment (start 124.46 114.3) (end 124.46 110.49) (width 1) (layer F.Cu) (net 7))
 (segment (start 116.84 121.92) (end 124.46 114.3) (width 1) (layer F.Cu) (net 7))
 (segment (start 124.46 110.49) (end 124.46 102.87) (width 1) (layer F.Cu) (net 7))
 (segment (start 126.492 100.838) (end 129.032 100.838) (width 1) (layer F.Cu) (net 7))
 (segment (start 124.46 102.87) (end 126.492 100.838) (width 1) (layer F.Cu) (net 7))
 (segment (start 118.872 106.128) (end 115 110) (width 1) (layer F.Cu) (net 8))
 (segment (start 118.872 105.918) (end 118.872 106.128) (width 1) (layer F.Cu) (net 8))
 (segment (start 101.6 127) (end 101.6 130.81) (width 1) (layer F.Cu) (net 8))
 (segment (start 105.41 125.73) (end 105.41 124.46) (width 0.4) (layer F.Cu) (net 8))
 (segment (start 105.41 124.46) (end 104.14 123.19) (width 0.4) (layer F.Cu) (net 8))
 (segment (start 104.14 123.19) (end 104.14 113.03) (width 0.4) (layer F.Cu) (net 8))
 (segment (start 107.17 110) (end 115 110) (width 1) (layer F.Cu) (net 8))
 (segment (start 104.14 113.03) (end 107.17 110) (width 1) (layer F.Cu) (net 8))
 (segment (start 101.6 130.81) (end 101.6 132.08) (width 1) (layer F.Cu) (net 8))
 (segment (start 101.6 132.08) (end 102.87 133.35) (width 1) (layer F.Cu) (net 8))
 (segment (start 102.87 133.35) (end 104.14 133.35) (width 1) (layer F.Cu) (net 8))
 (segment (start 104.14 133.35) (end 105.41 132.08) (width 1) (layer F.Cu) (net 8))
 (segment (start 105.41 132.08) (end 105.41 125.73) (width 1) (layer F.Cu) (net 8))
 (segment (start 90 118.5) (end 95.47 113.03) (width 1) (layer F.Cu) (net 12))
 (segment (start 90 120) (end 90 118.5) (width 1) (layer F.Cu) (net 12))
 (segment (start 95.47 107.73) (end 97.79 105.41) (width 1) (layer F.Cu) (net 12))
 (segment (start 95.47 113.03) (end 95.47 107.73) (width 1) (layer F.Cu) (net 12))
 (segment (start 95.47 113.03) (end 95.47 118.33) (width 1) (layer F.Cu) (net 12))
 (segment (start 99.06 121.92) (end 101.6 121.92) (width 1) (layer F.Cu) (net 12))
 (segment (start 95.47 118.33) (end 99.06 121.92) (width 1) (layer F.Cu) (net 12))
 (segment (start 87.63 105.41) (end 90.17 102.87) (width 1) (layer F.Cu) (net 6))
 (segment (start 83.82 105.41) (end 87.63 105.41) (width 1) (layer F.Cu) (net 6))
 (segment (start 91.30199 101.73801) (end 91.73801 101.73801) (width 0.4) (layer F.Cu) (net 6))
 (segment (start 90.17 102.87) (end 91.30199 101.73801) (width 0.4) (layer F.Cu) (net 6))
 (segment (start 91.73801 101.73801) (end 94 104) (width 0.4) (layer F.Cu) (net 6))
 (segment (start 94 104) (end 96 104) (width 0.4) (layer F.Cu) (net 6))
 (segment (start 96 104) (end 96.622 103.378) (width 0.4) (layer F.Cu) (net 6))
 (segment (start 96.622 103.378) (end 103.378 103.378) (width 0.4) (layer F.Cu) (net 6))
 (segment (start 103.378 103.378) (end 118.872 103.378) (width 1) (layer F.Cu) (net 6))
 (segment (start 134.62 86.36) (end 135.89 87.63) (width 0.4) (layer F.Cu) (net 6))
 (segment (start 132.08 86.36) (end 134.62 86.36) (width 0.4) (layer F.Cu) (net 6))
 (segment (start 132.08 86.36) (end 129.54 88.9) (width 0.4) (layer F.Cu) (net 6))
 (segment (start 129.54 88.9) (end 129.54 93.98) (width 0.4) (layer F.Cu) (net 6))
 (segment (start 129.54 93.98) (end 132.08 96.52) (width 0.4) (layer F.Cu) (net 6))
 (segment (start 132.08 96.52) (end 134.62 96.52) (width 0.4) (layer F.Cu) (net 6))
 (segment (start 144.78 88.9) (end 137.16 88.9) (width 1) (layer F.Cu) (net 1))
 (segment (start 116.84 82.55) (end 138.43 82.55) (width 1) (layer F.Cu) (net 1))
 (segment (start 138.43 82.55) (end 144.78 88.9) (width 1) (layer F.Cu) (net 1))
 (segment (start 118.11 81.28) (end 116.84 82.55) (width 1) (layer F.Cu) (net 1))
 (segment (start 118.11 72.39) (end 118.11 81.28) (width 1) (layer F.Cu) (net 1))
 (segment (start 83.82 93.98) (end 83.82 97.79) (width 1) (layer F.Cu) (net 2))
 (segment (start 116.84 67.31) (end 110.49 67.31) (width 1) (layer F.Cu) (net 2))
 (segment (start 110.49 67.31) (end 83.82 93.98) (width 1) (layer F.Cu) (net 2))
 (segment (start 123.19 67.31) (end 129.54 73.66) (width 1) (layer F.Cu) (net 2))
 (segment (start 116.84 67.97) (end 117.5 67.31) (width 0.4) (layer F.Cu) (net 2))
 (segment (start 116.84 71.12) (end 116.84 67.97) (width 0.4) (layer F.Cu) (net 2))
 (segment (start 116.84 67.31) (end 117.5 67.31) (width 1) (layer F.Cu) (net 2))
 (segment (start 117.5 67.31) (end 123.19 67.31) (width 1) (layer F.Cu) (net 2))
 (segment (start 121.412 89.408) (end 121.92 88.9) (width 1) (layer F.Cu) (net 10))
 (segment (start 117.602 89.408) (end 121.412 89.408) (width 1) (layer F.Cu) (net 10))
 (segment (start 87.63 124.46) (end 101.6 124.46) (width 1) (layer F.Cu) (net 11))
 (segment (start 83.82 120.65) (end 87.63 124.46) (width 1) (layer F.Cu) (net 11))
 (segment (start 90.17 110.49) (end 83.82 116.84) (width 1) (layer F.Cu) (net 11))
 (segment (start 83.82 116.84) (end 83.82 120.65) (width 1) (layer F.Cu) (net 11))
 (segment (start 142.24 100.1) (end 141.2 99.06) (width 1) (layer F.Cu) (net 13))
 (segment (start 142.24 101.6) (end 142.24 100.1) (width 1) (layer F.Cu) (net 13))
 (segment (start 138.432806 99.06) (end 135.52001 96.147204) (width 1) (layer F.Cu) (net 13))
 (segment (start 135.52001 96.147204) (end 135.256403 95.883597) (width 1) (layer F.Cu) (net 13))
 (segment (start 141.2 99.06) (end 138.432806 99.06) (width 1) (layer F.Cu) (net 13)))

